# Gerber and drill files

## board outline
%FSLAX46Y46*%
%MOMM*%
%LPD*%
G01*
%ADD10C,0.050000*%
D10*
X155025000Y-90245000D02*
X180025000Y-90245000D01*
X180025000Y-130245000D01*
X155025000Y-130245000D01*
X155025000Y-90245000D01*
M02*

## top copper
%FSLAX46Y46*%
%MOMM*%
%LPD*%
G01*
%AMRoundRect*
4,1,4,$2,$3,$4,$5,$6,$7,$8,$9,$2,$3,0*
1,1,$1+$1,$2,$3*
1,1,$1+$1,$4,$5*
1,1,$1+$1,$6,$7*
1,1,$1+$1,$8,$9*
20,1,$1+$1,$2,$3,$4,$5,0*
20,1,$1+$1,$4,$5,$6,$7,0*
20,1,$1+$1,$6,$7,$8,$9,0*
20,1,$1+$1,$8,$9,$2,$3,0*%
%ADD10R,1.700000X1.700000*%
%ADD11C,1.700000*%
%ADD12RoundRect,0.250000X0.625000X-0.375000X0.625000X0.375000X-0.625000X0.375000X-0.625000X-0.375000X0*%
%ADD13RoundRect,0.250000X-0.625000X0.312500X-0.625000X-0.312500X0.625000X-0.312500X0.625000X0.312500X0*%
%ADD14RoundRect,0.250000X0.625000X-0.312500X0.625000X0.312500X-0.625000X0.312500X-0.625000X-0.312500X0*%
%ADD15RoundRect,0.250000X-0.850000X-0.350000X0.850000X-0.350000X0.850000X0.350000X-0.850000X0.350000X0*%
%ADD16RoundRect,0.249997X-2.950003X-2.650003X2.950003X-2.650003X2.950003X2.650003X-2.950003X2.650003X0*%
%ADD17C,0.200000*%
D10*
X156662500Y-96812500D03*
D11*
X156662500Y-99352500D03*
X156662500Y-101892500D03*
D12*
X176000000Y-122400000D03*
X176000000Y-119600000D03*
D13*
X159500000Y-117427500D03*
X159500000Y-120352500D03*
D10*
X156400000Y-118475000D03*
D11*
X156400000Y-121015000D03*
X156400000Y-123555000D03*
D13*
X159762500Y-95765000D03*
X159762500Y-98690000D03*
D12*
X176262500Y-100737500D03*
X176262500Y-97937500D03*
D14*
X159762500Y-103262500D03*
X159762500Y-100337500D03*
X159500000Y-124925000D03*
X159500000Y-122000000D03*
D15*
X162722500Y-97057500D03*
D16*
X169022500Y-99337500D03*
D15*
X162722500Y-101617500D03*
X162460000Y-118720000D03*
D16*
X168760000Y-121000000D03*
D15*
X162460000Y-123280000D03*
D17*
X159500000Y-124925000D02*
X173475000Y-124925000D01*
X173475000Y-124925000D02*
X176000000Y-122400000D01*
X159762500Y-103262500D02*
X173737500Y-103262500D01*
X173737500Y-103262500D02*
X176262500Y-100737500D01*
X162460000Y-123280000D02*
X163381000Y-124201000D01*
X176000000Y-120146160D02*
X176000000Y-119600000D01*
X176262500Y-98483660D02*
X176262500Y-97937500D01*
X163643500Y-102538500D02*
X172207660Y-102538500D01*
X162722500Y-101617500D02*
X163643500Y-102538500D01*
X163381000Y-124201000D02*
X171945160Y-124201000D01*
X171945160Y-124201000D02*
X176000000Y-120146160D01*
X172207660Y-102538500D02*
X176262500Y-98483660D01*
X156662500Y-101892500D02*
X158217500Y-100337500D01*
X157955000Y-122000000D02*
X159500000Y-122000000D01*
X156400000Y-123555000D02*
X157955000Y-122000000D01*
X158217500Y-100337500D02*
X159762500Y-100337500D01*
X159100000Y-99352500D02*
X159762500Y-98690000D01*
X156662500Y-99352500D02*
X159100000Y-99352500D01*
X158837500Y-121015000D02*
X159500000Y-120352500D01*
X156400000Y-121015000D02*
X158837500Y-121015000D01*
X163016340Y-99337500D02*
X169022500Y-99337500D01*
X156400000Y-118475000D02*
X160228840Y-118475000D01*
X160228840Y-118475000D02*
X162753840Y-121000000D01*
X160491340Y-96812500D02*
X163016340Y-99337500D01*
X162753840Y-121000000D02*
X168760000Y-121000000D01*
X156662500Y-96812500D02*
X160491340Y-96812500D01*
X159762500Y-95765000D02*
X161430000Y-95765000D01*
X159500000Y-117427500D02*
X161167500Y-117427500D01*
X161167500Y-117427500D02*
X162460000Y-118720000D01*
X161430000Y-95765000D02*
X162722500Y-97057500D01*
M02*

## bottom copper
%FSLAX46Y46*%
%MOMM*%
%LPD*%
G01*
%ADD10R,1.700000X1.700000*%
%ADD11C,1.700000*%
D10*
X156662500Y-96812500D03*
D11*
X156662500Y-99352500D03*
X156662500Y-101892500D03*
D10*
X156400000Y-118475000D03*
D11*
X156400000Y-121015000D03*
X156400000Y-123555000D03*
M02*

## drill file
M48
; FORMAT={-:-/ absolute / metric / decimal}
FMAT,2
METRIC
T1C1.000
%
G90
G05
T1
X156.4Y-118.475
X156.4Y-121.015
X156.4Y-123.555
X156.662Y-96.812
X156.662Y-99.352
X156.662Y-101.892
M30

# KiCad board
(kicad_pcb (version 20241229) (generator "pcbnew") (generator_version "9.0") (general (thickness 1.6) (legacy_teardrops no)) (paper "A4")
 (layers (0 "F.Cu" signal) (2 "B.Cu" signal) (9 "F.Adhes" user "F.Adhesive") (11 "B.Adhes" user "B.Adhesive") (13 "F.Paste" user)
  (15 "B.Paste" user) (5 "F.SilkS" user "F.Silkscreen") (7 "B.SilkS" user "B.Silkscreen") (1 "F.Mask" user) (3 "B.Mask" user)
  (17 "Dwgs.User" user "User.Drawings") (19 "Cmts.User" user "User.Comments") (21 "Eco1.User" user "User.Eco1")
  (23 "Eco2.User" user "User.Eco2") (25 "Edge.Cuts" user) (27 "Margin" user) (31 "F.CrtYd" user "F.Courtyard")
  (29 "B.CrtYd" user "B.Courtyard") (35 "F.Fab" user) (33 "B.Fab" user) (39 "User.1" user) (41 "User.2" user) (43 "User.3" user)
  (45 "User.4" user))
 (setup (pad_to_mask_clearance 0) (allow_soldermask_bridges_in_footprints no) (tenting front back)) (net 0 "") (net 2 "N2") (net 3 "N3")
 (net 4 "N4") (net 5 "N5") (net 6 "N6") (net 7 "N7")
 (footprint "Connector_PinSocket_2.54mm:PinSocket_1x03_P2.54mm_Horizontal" (layer "F.Cu") (at 156.6625 96.8125)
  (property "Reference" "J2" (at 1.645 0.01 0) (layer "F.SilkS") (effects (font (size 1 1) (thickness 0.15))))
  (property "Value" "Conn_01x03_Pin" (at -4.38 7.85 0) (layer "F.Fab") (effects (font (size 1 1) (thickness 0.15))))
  (pad "1" thru_hole rect (at 0 0) (size 1.7 1.7) (drill 1) (layers "*.Cu" "*.Mask") (remove_unused_layers no) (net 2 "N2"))
  (pad "2" thru_hole circle (at 0 2.54) (size 1.7 1.7) (drill 1) (layers "*.Cu" "*.Mask") (remove_unused_layers no) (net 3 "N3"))
  (pad "3" thru_hole circle (at 0 5.08) (size 1.7 1.7) (drill 1) (layers "*.Cu" "*.Mask") (remove_unused_layers no) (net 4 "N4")))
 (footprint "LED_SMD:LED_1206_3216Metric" (layer "F.Cu") (at 176 121 90)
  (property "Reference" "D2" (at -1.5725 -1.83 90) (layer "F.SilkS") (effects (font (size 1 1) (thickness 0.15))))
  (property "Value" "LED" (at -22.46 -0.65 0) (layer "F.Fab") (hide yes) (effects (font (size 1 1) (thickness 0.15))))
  (pad "1" smd roundrect (at -1.4 0 90) (size 1.25 1.75) (layers "F.Cu" "F.Mask" "F.Paste") (roundrect_rratio 0.2) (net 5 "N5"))
  (pad "2" smd roundrect (at 1.4 0 90) (size 1.25 1.75) (layers "F.Cu" "F.Mask" "F.Paste") (roundrect_rratio 0.2) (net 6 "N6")))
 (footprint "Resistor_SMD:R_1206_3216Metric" (layer "F.Cu") (at 159.5 118.89 -90)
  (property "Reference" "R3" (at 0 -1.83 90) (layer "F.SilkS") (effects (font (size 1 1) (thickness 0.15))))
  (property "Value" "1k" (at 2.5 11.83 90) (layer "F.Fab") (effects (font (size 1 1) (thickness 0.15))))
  (pad "1" smd roundrect (at -1.4625 0 270) (size 1.125 1.75) (layers "F.Cu" "F.Mask" "F.Paste") (roundrect_rratio 0.222222) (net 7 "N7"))
  (pad "2" smd roundrect (at 1.4625 0 270) (size 1.125 1.75) (layers "F.Cu" "F.Mask" "F.Paste") (roundrect_rratio 0.222222) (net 3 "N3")))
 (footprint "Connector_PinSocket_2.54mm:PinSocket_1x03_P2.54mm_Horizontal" (layer "F.Cu") (at 156.4 118.475)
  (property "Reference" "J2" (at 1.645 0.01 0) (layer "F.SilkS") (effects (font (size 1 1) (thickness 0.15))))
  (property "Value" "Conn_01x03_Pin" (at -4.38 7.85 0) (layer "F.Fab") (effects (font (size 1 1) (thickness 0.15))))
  (pad "1" thru_hole rect (at 0 0) (size 1.7 1.7) (drill 1) (layers "*.Cu" "*.Mask") (remove_unused_layers no) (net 2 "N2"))
  (pad "2" thru_hole circle (at 0 2.54) (size 1.7 1.7) (drill 1) (layers "*.Cu" "*.Mask") (remove_unused_layers no) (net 3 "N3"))
  (pad "3" thru_hole circle (at 0 5.08) (size 1.7 1.7) (drill 1) (layers "*.Cu" "*.Mask") (remove_unused_layers no) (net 4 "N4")))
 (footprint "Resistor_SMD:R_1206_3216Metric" (layer "F.Cu") (at 159.7625 97.2275 -90)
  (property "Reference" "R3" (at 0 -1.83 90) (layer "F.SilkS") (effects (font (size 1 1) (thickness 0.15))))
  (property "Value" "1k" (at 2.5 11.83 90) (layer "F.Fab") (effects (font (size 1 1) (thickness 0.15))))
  (pad "1" smd roundrect (at -1.4625 0 270) (size 1.125 1.75) (layers "F.Cu" "F.Mask" "F.Paste") (roundrect_rratio 0.222222) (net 7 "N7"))
  (pad "2" smd roundrect (at 1.4625 0 270) (size 1.125 1.75) (layers "F.Cu" "F.Mask" "F.Paste") (roundrect_rratio 0.222222) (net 3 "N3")))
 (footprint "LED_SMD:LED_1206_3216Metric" (layer "F.Cu") (at 176.2625 99.3375 90)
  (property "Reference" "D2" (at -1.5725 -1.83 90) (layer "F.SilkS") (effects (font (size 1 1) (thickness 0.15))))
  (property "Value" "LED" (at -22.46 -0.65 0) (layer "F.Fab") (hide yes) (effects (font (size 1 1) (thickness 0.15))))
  (pad "1" smd roundrect (at -1.4 0 90) (size 1.25 1.75) (layers "F.Cu" "F.Mask" "F.Paste") (roundrect_rratio 0.2) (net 5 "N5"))
  (pad "2" smd roundrect (at 1.4 0 90) (size 1.25 1.75) (layers "F.Cu" "F.Mask" "F.Paste") (roundrect_rratio 0.2) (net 6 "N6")))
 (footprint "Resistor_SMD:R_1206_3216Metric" (layer "F.Cu") (at 159.7625 101.8 90)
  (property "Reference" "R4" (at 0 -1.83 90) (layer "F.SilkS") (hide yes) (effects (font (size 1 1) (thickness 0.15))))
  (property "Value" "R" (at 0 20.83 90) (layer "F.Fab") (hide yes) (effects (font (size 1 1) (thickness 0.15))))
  (pad "1" smd roundrect (at -1.4625 0 90) (size 1.125 1.75) (layers "F.Cu" "F.Mask" "F.Paste") (roundrect_rratio 0.222222) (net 5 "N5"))
  (pad "2" smd roundrect (at 1.4625 0 90) (size 1.125 1.75) (layers "F.Cu" "F.Mask" "F.Paste") (roundrect_rratio 0.222222) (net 4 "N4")))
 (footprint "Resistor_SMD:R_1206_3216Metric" (layer "F.Cu") (at 159.5 123.4625 90)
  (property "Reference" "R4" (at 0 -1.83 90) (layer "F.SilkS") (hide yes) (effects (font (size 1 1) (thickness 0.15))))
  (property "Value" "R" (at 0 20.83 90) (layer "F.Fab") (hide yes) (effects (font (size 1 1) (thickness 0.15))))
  (pad "1" smd roundrect (at -1.4625 0 90) (size 1.125 1.75) (layers "F.Cu" "F.Mask" "F.Paste") (roundrect_rratio 0.222222) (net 5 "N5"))
  (pad "2" smd roundrect (at 1.4625 0 90) (size 1.125 1.75) (layers "F.Cu" "F.Mask" "F.Paste") (roundrect_rratio 0.222222) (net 4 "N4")))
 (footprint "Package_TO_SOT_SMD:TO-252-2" (layer "F.Cu") (at 167.7625 99.3375)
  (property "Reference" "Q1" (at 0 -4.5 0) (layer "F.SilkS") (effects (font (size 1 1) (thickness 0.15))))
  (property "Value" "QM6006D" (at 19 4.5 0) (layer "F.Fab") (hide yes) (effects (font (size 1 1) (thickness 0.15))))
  (pad "" smd roundrect (at -0.415 -1.525) (size 3.05 2.75) (layers "F.Paste") (roundrect_rratio 0.090909))
  (pad "" smd roundrect (at -0.415 1.525) (size 3.05 2.75) (layers "F.Paste") (roundrect_rratio 0.090909))
  (pad "" smd roundrect (at 2.935 -1.525) (size 3.05 2.75) (layers "F.Paste") (roundrect_rratio 0.090909))
  (pad "" smd roundrect (at 2.935 1.525) (size 3.05 2.75) (layers "F.Paste") (roundrect_rratio 0.090909))
  (pad "1" smd roundrect (at -5.04 -2.28) (size 2.2 1.2) (layers "F.Cu" "F.Mask" "F.Paste") (roundrect_rratio 0.208333) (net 7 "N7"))
  (pad "2" smd roundrect (at 1.26 0) (size 6.4 5.8) (layers "F.Cu" "F.Mask") (roundrect_rratio 0.043103) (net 2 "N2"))
  (pad "3" smd roundrect (at -5.04 2.28) (size 2.2 1.2) (layers "F.Cu" "F.Mask" "F.Paste") (roundrect_rratio 0.208333) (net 6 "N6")))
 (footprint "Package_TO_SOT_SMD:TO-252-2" (layer "F.Cu") (at 167.5 121)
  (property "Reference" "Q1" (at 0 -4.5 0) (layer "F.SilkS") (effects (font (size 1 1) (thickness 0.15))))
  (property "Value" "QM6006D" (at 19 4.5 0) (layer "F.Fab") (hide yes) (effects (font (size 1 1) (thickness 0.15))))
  (pad "" smd roundrect (at -0.415 -1.525) (size 3.05 2.75) (layers "F.Paste") (roundrect_rratio 0.090909))
  (pad "" smd roundrect (at -0.415 1.525) (size 3.05 2.75) (layers "F.Paste") (roundrect_rratio 0.090909))
  (pad "" smd roundrect (at 2.935 -1.525) (size 3.05 2.75) (layers "F.Paste") (roundrect_rratio 0.090909))
  (pad "" smd roundrect (at 2.935 1.525) (size 3.05 2.75) (layers "F.Paste") (roundrect_rratio 0.090909))
  (pad "1" smd roundrect (at -5.04 -2.28) (size 2.2 1.2) (layers "F.Cu" "F.Mask" "F.Paste") (roundrect_rratio 0.208333) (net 7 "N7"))
  (pad "2" smd roundrect (at 1.26 0) (size 6.4 5.8) (layers "F.Cu" "F.Mask") (roundrect_rratio 0.043103) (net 2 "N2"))
  (pad "3" smd roundrect (at -5.04 2.28) (size 2.2 1.2) (layers "F.Cu" "F.Mask" "F.Paste") (roundrect_rratio 0.208333) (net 6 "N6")))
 (gr_rect (start 155.025 90.245) (end 180.025 130.245) (stroke (width 0.05) (type default)) (fill no) (layer "Edge.Cuts"))
 (segment (start 159.5 124.925) (end 173.475 124.925) (width 0.2) (layer "F.Cu") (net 5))
 (segment (start 173.475 124.925) (end 176 122.4) (width 0.2) (layer "F.Cu") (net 5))
 (segment (start 159.7625 103.2625) (end 173.7375 103.2625) (width 0.2) (layer "F.Cu") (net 5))
 (segment (start 173.7375 103.2625) (end 176.2625 100.7375) (width 0.2) (layer "F.Cu") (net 5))
 (segment (start 162.46 123.28) (end 163.381 124.201) (width 0.2) (layer "F.Cu") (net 6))
 (segment (start 176 120.14616) (end 176 119.6) (width 0.2) (layer "F.Cu") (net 6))
 (segment (start 176.2625 98.48366) (end 176.2625 97.9375) (width 0.2) (layer "F.Cu") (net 6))
 (segment (start 163.6435 102.5385) (end 172.20766 102.5385) (width 0.2) (layer "F.Cu") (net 6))
 (segment (start 162.7225 101.6175) (end 163.6435 102.5385) (width 0.2) (layer "F.Cu") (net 6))
 (segment (start 163.381 124.201) (end 171.94516 124.201) (width 0.2) (layer "F.Cu") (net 6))
 (segment (start 171.94516 124.201) (end 176 120.14616) (width 0.2) (layer "F.Cu") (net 6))
 (segment (start 172.20766 102.5385) (end 176.2625 98.48366) (width 0.2) (layer "F.Cu") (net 6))
 (segment (start 156.6625 101.8925) (end 158.2175 100.3375) (width 0.2) (layer "F.Cu") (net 4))
 (segment (start 157.955 122) (end 159.5 122) (width 0.2) (layer "F.Cu") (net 4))
 (segment (start 156.4 123.555) (end 157.955 122) (width 0.2) (layer "F.Cu") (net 4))
 (segment (start 158.2175 100.3375) (end 159.7625 100.3375) (width 0.2) (layer "F.Cu") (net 4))
 (segment (start 159.1 99.3525) (end 159.7625 98.69) (width 0.2) (layer "F.Cu") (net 3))
 (segment (start 156.6625 99.3525) (end 159.1 99.3525) (width 0.2) (layer "F.Cu") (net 3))
 (segment (start 158.8375 121.015) (end 159.5 120.3525) (width 0.2) (layer "F.Cu") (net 3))
 (segment (start 156.4 121.015) (end 158.8375 121.015) (width 0.2) (layer "F.Cu") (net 3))
 (segment (start 163.01634 99.3375) (end 169.0225 99.3375) (width 0.2) (layer "F.Cu") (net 2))
 (segment (start 156.4 118.475) (end 160.22884 118.475) (width 0.2) (layer "F.Cu") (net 2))
 (segment (start 160.22884 118.475) (end 162.75384 121) (width 0.2) (layer "F.Cu") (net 2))
 (segment (start 160.49134 96.8125) (end 163.01634 99.3375) (width 0.2) (layer "F.Cu") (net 2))
 (segment (start 162.75384 121) (end 168.76 121) (width 0.2) (layer "F.Cu") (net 2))
 (segment (start 156.6625 96.8125) (end 160.49134 96.8125) (width 0.2) (layer "F.Cu") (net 2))
 (segment (start 159.7625 95.765) (end 161.43 95.765) (width 0.2) (layer "F.Cu") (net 7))
 (segment (start 159.5 117.4275) (end 161.1675 117.4275) (width 0.2) (layer "F.Cu") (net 7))
 (segment (start 161.1675 117.4275) (end 162.46 118.72) (width 0.2) (layer "F.Cu") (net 7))
 (segment (start 161.43 95.765) (end 162.7225 97.0575) (width 0.2) (layer "F.Cu") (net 7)))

